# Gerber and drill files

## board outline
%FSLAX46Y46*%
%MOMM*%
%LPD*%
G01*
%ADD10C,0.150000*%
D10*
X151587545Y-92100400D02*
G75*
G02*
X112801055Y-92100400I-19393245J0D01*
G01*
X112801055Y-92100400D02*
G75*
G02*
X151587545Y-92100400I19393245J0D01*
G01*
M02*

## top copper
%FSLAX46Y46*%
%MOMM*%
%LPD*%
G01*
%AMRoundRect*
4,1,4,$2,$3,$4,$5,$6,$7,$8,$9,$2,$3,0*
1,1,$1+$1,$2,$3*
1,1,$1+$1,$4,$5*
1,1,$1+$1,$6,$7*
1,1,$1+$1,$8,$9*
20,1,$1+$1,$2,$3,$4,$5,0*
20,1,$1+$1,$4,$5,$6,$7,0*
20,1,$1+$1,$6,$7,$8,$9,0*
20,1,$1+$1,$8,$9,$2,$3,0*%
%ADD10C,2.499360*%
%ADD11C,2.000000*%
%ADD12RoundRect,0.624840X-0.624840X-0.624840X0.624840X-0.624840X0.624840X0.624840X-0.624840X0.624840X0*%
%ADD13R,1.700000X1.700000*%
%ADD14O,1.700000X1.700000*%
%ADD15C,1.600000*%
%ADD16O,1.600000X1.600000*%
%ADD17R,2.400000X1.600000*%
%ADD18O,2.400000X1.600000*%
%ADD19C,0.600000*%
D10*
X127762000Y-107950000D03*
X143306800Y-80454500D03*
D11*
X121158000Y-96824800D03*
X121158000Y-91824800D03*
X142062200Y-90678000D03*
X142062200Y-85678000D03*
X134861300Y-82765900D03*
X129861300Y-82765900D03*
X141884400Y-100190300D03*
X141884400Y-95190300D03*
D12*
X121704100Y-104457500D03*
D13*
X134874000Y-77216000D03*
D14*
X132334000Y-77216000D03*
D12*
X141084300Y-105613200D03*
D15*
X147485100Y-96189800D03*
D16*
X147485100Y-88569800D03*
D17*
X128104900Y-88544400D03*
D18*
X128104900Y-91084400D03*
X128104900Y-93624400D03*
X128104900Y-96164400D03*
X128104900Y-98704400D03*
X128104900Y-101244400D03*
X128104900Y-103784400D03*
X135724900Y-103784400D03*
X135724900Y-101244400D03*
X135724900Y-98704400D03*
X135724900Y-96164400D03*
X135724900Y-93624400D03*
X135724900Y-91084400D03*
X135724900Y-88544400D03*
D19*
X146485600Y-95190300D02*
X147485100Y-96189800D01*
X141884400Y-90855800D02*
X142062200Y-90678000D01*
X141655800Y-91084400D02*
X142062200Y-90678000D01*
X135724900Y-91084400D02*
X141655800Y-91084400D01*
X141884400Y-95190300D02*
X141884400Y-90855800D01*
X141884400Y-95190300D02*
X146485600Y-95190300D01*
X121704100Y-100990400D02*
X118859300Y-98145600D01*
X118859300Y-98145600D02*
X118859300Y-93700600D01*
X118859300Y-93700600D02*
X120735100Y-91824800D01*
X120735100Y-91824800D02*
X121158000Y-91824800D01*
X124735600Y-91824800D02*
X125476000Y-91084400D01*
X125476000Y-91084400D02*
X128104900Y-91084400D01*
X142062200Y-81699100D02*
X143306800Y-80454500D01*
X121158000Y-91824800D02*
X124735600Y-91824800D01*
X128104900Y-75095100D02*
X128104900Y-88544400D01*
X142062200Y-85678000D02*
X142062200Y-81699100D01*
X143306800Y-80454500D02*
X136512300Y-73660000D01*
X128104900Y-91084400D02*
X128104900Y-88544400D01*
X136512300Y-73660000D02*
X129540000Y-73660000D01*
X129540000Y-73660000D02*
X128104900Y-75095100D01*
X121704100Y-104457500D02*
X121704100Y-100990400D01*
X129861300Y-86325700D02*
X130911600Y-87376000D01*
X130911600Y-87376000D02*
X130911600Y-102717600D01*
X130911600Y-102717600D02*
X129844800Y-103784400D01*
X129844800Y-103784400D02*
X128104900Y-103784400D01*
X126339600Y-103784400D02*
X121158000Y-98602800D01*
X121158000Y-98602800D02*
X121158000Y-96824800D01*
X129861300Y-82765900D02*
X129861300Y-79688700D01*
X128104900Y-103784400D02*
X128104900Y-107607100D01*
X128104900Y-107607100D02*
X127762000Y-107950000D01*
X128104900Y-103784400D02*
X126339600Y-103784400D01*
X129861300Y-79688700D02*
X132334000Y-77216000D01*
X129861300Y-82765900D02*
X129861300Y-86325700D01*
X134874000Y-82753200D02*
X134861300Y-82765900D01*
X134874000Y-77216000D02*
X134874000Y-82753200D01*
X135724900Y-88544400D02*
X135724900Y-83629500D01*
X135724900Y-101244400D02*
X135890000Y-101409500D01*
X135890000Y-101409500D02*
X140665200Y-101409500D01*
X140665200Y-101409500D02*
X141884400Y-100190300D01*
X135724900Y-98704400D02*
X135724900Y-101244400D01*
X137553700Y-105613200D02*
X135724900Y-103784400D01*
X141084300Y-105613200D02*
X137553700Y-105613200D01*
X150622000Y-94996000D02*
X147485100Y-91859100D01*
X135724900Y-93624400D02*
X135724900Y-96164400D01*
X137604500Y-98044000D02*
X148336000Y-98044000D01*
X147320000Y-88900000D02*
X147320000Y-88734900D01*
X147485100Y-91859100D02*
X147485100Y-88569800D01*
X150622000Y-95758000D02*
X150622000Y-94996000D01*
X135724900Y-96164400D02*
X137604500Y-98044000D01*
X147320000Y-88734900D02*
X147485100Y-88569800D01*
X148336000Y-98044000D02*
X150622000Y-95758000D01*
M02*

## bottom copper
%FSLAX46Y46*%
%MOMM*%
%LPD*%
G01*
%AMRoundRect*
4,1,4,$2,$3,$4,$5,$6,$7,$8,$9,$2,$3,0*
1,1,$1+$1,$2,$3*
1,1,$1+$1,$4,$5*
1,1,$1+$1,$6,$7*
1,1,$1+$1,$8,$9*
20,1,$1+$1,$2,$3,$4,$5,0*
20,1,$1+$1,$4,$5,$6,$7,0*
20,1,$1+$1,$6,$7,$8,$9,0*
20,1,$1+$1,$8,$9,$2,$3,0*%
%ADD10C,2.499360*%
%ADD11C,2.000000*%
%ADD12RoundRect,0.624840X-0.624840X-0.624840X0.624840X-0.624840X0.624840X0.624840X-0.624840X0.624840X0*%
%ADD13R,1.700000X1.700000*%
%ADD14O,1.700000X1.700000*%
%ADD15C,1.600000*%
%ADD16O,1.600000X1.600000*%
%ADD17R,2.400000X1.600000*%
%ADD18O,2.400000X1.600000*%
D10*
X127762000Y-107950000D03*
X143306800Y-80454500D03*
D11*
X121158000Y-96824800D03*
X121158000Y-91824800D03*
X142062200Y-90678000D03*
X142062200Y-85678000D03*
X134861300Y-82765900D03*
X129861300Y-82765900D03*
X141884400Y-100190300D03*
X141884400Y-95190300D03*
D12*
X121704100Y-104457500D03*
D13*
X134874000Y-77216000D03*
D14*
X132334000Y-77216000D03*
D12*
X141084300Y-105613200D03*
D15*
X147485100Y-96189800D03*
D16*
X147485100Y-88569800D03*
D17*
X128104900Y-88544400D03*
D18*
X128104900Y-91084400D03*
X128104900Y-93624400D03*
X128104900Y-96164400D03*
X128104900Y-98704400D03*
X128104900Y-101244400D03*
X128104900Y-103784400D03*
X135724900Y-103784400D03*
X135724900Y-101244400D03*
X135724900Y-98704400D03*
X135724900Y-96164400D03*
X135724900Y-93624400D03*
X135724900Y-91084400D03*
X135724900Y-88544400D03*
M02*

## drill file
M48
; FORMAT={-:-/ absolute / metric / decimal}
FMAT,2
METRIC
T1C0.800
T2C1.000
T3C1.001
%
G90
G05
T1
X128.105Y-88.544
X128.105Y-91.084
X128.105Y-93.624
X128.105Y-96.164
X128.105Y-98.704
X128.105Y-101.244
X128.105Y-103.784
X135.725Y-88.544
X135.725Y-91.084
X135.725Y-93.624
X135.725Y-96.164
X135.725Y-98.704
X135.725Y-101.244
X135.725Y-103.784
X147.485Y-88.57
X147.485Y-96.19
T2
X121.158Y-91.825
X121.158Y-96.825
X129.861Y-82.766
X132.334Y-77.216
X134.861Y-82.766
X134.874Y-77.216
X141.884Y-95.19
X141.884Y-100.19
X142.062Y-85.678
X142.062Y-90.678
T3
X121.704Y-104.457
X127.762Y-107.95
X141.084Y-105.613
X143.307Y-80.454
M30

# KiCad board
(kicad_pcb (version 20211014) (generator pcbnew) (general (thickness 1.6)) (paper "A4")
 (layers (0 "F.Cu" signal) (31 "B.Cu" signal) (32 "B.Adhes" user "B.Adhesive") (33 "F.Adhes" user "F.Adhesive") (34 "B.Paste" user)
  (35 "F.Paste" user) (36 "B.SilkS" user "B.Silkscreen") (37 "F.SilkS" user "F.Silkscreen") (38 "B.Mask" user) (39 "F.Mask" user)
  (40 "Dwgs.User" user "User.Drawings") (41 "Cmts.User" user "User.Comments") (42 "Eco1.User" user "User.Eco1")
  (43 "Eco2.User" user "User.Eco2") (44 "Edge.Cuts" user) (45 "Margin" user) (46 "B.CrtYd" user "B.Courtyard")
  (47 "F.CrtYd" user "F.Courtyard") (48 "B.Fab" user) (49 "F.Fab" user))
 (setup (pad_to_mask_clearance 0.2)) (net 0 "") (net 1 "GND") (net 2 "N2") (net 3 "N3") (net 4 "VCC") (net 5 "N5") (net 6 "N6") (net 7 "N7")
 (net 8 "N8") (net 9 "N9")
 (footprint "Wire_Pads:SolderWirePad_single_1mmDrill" (layer "F.Cu") (at 127.762 107.95)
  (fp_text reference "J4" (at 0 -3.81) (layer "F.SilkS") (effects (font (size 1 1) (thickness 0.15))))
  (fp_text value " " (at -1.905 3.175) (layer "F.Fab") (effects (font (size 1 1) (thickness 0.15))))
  (pad "1" thru_hole circle locked (at 0 0) (size 2.49936 2.49936) (drill 1.00076) (layers *.Cu *.Mask) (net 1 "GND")))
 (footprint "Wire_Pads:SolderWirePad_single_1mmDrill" (layer "F.Cu") (at 143.3068 80.4545)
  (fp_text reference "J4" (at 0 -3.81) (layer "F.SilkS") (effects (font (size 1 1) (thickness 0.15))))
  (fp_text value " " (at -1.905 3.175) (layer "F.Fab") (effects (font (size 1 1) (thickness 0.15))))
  (pad "1" thru_hole circle locked (at 0 0) (size 2.49936 2.49936) (drill 1.00076) (layers *.Cu *.Mask) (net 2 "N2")))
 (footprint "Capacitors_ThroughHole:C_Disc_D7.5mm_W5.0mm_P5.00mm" (layer "F.Cu") (at 121.158 96.8248 90)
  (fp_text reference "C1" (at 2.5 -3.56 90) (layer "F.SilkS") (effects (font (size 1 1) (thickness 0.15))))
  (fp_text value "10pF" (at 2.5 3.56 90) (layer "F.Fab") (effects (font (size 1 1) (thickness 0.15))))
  (pad "1" thru_hole circle locked (at 0 0 90) (size 2 2) (drill 1) (layers *.Cu *.Mask) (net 1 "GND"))
  (pad "2" thru_hole circle locked (at 5 0 90) (size 2 2) (drill 1) (layers *.Cu *.Mask) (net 2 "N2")))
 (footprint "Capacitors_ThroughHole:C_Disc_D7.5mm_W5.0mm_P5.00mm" (layer "F.Cu") (at 142.0622 90.678 90)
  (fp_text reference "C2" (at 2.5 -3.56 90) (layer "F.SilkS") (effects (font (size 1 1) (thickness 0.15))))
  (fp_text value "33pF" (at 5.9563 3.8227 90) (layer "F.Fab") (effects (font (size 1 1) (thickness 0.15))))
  (pad "1" thru_hole circle locked (at 0 0 90) (size 2 2) (drill 1) (layers *.Cu *.Mask) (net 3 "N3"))
  (pad "2" thru_hole circle locked (at 5 0 90) (size 2 2) (drill 1) (layers *.Cu *.Mask) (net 2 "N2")))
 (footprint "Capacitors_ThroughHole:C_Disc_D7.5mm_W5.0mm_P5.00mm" (layer "F.Cu") (at 134.8613 82.7659 180)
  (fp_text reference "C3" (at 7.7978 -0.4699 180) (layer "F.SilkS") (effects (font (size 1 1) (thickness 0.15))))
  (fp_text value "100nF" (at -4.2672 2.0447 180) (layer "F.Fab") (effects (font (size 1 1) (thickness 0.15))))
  (pad "1" thru_hole circle locked (at 0 0 180) (size 2 2) (drill 1) (layers *.Cu *.Mask) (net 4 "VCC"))
  (pad "2" thru_hole circle locked (at 5 0 180) (size 2 2) (drill 1) (layers *.Cu *.Mask) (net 1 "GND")))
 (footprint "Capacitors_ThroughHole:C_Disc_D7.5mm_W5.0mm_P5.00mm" (layer "F.Cu") (at 141.8844 100.1903 90)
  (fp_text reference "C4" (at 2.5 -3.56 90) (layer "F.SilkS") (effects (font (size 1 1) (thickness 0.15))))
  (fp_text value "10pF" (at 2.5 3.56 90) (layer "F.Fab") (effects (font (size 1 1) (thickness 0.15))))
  (pad "1" thru_hole circle locked (at 0 0 90) (size 2 2) (drill 1) (layers *.Cu *.Mask) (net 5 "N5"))
  (pad "2" thru_hole circle locked (at 5 0 90) (size 2 2) (drill 1) (layers *.Cu *.Mask) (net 3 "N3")))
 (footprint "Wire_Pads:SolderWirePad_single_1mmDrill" (layer "F.Cu") (at 121.7041 104.4575)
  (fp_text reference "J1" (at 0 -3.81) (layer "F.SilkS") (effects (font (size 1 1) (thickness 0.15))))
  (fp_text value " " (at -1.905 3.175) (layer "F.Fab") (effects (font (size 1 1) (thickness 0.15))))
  (pad "1" thru_hole roundrect locked (at 0 0) (size 2.49936 2.49936) (drill 1.00076) (layers *.Cu *.Mask) (roundrect_rratio 0.25)
   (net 2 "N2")))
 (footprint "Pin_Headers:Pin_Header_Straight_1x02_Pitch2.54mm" (layer "F.Cu") (at 134.874 77.216 -90)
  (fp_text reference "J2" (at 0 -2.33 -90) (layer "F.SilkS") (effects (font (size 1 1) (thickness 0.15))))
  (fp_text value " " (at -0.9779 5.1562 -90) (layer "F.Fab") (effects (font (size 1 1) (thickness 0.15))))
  (pad "1" thru_hole rect locked (at 0 0 270) (size 1.7 1.7) (drill 1) (layers *.Cu *.Mask) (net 4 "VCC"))
  (pad "2" thru_hole oval locked (at 0 2.54 270) (size 1.7 1.7) (drill 1) (layers *.Cu *.Mask) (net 1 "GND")))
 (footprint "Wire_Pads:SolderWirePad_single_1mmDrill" (layer "F.Cu") (at 141.0843 105.6132)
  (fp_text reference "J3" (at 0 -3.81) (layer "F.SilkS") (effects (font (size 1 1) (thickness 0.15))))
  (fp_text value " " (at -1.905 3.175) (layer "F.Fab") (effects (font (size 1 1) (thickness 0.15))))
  (pad "1" thru_hole roundrect locked (at 0 0) (size 2.49936 2.49936) (drill 1.00076) (layers *.Cu *.Mask) (roundrect_rratio 0.25)
   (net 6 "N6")))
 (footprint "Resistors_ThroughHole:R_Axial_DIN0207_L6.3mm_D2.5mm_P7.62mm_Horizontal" (layer "F.Cu") (at 147.4851 96.1898 90)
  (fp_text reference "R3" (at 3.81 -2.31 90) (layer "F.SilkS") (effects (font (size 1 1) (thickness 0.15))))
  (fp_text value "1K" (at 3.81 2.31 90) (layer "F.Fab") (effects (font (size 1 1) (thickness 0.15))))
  (pad "1" thru_hole circle locked (at 0 0 90) (size 1.6 1.6) (drill 0.8) (layers *.Cu *.Mask) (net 3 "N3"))
  (pad "2" thru_hole oval locked (at 7.62 0 90) (size 1.6 1.6) (drill 0.8) (layers *.Cu *.Mask) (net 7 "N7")))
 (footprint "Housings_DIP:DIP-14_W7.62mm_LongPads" (layer "F.Cu") (at 128.1049 88.5444)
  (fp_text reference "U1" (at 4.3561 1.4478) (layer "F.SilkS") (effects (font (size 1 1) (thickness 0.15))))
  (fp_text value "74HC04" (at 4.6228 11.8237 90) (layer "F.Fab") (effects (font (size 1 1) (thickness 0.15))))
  (pad "1" thru_hole rect locked (at 0 0) (size 2.4 1.6) (drill 0.8) (layers *.Cu *.Mask) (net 2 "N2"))
  (pad "2" thru_hole oval locked (at 0 2.54) (size 2.4 1.6) (drill 0.8) (layers *.Cu *.Mask) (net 2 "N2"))
  (pad "3" thru_hole oval locked (at 0 5.08) (size 2.4 1.6) (drill 0.8) (layers *.Cu *.Mask) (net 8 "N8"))
  (pad "4" thru_hole oval locked (at 0 7.62) (size 2.4 1.6) (drill 0.8) (layers *.Cu *.Mask) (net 8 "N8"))
  (pad "5" thru_hole oval locked (at 0 10.16) (size 2.4 1.6) (drill 0.8) (layers *.Cu *.Mask) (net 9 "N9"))
  (pad "6" thru_hole oval locked (at 0 12.7) (size 2.4 1.6) (drill 0.8) (layers *.Cu *.Mask) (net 9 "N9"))
  (pad "7" thru_hole oval locked (at 0 15.24) (size 2.4 1.6) (drill 0.8) (layers *.Cu *.Mask) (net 1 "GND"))
  (pad "8" thru_hole oval locked (at 7.62 15.24) (size 2.4 1.6) (drill 0.8) (layers *.Cu *.Mask) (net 6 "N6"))
  (pad "9" thru_hole oval locked (at 7.62 12.7) (size 2.4 1.6) (drill 0.8) (layers *.Cu *.Mask) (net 5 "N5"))
  (pad "10" thru_hole oval locked (at 7.62 10.16) (size 2.4 1.6) (drill 0.8) (layers *.Cu *.Mask) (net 5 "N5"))
  (pad "11" thru_hole oval locked (at 7.62 7.62) (size 2.4 1.6) (drill 0.8) (layers *.Cu *.Mask) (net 7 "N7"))
  (pad "12" thru_hole oval locked (at 7.62 5.08) (size 2.4 1.6) (drill 0.8) (layers *.Cu *.Mask) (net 7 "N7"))
  (pad "13" thru_hole oval locked (at 7.62 2.54) (size 2.4 1.6) (drill 0.8) (layers *.Cu *.Mask) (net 3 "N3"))
  (pad "14" thru_hole oval locked (at 7.62 0) (size 2.4 1.6) (drill 0.8) (layers *.Cu *.Mask) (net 4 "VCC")))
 (gr_circle (center 132.1943 92.1004) (end 151.587545 92.1004) (layer "Edge.Cuts") (width 0.15) (fill none))
 (segment (start 146.4856 95.1903) (end 147.4851 96.1898) (width 0.6) (layer "F.Cu") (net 3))
 (segment (start 141.8844 90.8558) (end 142.0622 90.678) (width 0.6) (layer "F.Cu") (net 3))
 (segment (start 141.6558 91.0844) (end 142.0622 90.678) (width 0.6) (layer "F.Cu") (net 3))
 (segment (start 135.7249 91.0844) (end 141.6558 91.0844) (width 0.6) (layer "F.Cu") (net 3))
 (segment (start 141.8844 95.1903) (end 141.8844 90.8558) (width 0.6) (layer "F.Cu") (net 3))
 (segment (start 141.8844 95.1903) (end 146.4856 95.1903) (width 0.6) (layer "F.Cu") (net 3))
 (segment (start 121.7041 100.9904) (end 118.8593 98.1456) (width 0.6) (layer "F.Cu") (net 2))
 (segment (start 118.8593 98.1456) (end 118.8593 93.7006) (width 0.6) (layer "F.Cu") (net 2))
 (segment (start 118.8593 93.7006) (end 120.7351 91.8248) (width 0.6) (layer "F.Cu") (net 2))
 (segment (start 120.7351 91.8248) (end 121.158 91.8248) (width 0.6) (layer "F.Cu") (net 2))
 (segment (start 124.7356 91.8248) (end 125.476 91.0844) (width 0.6) (layer "F.Cu") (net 2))
 (segment (start 125.476 91.0844) (end 128.1049 91.0844) (width 0.6) (layer "F.Cu") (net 2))
 (segment (start 142.0622 81.6991) (end 143.3068 80.4545) (width 0.6) (layer "F.Cu") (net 2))
 (segment (start 121.158 91.8248) (end 124.7356 91.8248) (width 0.6) (layer "F.Cu") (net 2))
 (segment (start 128.1049 75.0951) (end 128.1049 88.5444) (width 0.6) (layer "F.Cu") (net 2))
 (segment (start 142.0622 85.678) (end 142.0622 81.6991) (width 0.6) (layer "F.Cu") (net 2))
 (segment (start 143.3068 80.4545) (end 136.5123 73.66) (width 0.6) (layer "F.Cu") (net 2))
 (segment (start 128.1049 91.0844) (end 128.1049 88.5444) (width 0.6) (layer "F.Cu") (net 2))
 (segment (start 136.5123 73.66) (end 129.54 73.66) (width 0.6) (layer "F.Cu") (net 2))
 (segment (start 129.54 73.66) (end 128.1049 75.0951) (width 0.6) (layer "F.Cu") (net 2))
 (segment (start 121.7041 104.4575) (end 121.7041 100.9904) (width 0.6) (layer "F.Cu") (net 2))
 (segment (start 129.8613 86.3257) (end 130.9116 87.376) (width 0.6) (layer "F.Cu") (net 1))
 (segment (start 130.9116 87.376) (end 130.9116 102.7176) (width 0.6) (layer "F.Cu") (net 1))
 (segment (start 130.9116 102.7176) (end 129.8448 103.7844) (width 0.6) (layer "F.Cu") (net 1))
 (segment (start 129.8448 103.7844) (end 128.1049 103.7844) (width 0.6) (layer "F.Cu") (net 1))
 (segment (start 126.3396 103.7844) (end 121.158 98.6028) (width 0.6) (layer "F.Cu") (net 1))
 (segment (start 121.158 98.6028) (end 121.158 96.8248) (width 0.6) (layer "F.Cu") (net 1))
 (segment (start 129.8613 82.7659) (end 129.8613 79.6887) (width 0.6) (layer "F.Cu") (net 1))
 (segment (start 128.1049 103.7844) (end 128.1049 107.6071) (width 0.6) (layer "F.Cu") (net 1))
 (segment (start 128.1049 107.6071) (end 127.762 107.95) (width 0.6) (layer "F.Cu") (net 1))
 (segment (start 128.1049 103.7844) (end 126.3396 103.7844) (width 0.6) (layer "F.Cu") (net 1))
 (segment (start 129.8613 79.6887) (end 132.334 77.216) (width 0.6) (layer "F.Cu") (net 1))
 (segment (start 129.8613 82.7659) (end 129.8613 86.3257) (width 0.6) (layer "F.Cu") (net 1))
 (segment (start 134.874 82.7532) (end 134.8613 82.7659) (width 0.6) (layer "F.Cu") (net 4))
 (segment (start 134.874 77.216) (end 134.874 82.7532) (width 0.6) (layer "F.Cu") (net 4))
 (segment (start 135.7249 88.5444) (end 135.7249 83.6295) (width 0.6) (layer "F.Cu") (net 4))
 (segment (start 135.7249 101.2444) (end 135.89 101.4095) (width 0.6) (layer "F.Cu") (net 5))
 (segment (start 135.89 101.4095) (end 140.6652 101.4095) (width 0.6) (layer "F.Cu") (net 5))
 (segment (start 140.6652 101.4095) (end 141.8844 100.1903) (width 0.6) (layer "F.Cu") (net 5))
 (segment (start 135.7249 98.7044) (end 135.7249 101.2444) (width 0.6) (layer "F.Cu") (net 5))
 (segment (start 137.5537 105.6132) (end 135.7249 103.7844) (width 0.6) (layer "F.Cu") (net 6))
 (segment (start 141.0843 105.6132) (end 137.5537 105.6132) (width 0.6) (layer "F.Cu") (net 6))
 (segment (start 150.622 94.996) (end 147.4851 91.8591) (width 0.6) (layer "F.Cu") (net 7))
 (segment (start 135.7249 93.6244) (end 135.7249 96.1644) (width 0.6) (layer "F.Cu") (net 7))
 (segment (start 137.6045 98.044) (end 148.336 98.044) (width 0.6) (layer "F.Cu") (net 7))
 (segment (start 147.32 88.9) (end 147.32 88.7349) (width 0.6) (layer "F.Cu") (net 7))
 (segment (start 147.4851 91.8591) (end 147.4851 88.5698) (width 0.6) (layer "F.Cu") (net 7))
 (segment (start 150.622 95.758) (end 150.622 94.996) (width 0.6) (layer "F.Cu") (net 7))
 (segment (start 135.7249 96.1644) (end 137.6045 98.044) (width 0.6) (layer "F.Cu") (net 7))
 (segment (start 147.32 88.7349) (end 147.4851 88.5698) (width 0.6) (layer "F.Cu") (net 7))
 (segment (start 148.336 98.044) (end 150.622 95.758) (width 0.6) (layer "F.Cu") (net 7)))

